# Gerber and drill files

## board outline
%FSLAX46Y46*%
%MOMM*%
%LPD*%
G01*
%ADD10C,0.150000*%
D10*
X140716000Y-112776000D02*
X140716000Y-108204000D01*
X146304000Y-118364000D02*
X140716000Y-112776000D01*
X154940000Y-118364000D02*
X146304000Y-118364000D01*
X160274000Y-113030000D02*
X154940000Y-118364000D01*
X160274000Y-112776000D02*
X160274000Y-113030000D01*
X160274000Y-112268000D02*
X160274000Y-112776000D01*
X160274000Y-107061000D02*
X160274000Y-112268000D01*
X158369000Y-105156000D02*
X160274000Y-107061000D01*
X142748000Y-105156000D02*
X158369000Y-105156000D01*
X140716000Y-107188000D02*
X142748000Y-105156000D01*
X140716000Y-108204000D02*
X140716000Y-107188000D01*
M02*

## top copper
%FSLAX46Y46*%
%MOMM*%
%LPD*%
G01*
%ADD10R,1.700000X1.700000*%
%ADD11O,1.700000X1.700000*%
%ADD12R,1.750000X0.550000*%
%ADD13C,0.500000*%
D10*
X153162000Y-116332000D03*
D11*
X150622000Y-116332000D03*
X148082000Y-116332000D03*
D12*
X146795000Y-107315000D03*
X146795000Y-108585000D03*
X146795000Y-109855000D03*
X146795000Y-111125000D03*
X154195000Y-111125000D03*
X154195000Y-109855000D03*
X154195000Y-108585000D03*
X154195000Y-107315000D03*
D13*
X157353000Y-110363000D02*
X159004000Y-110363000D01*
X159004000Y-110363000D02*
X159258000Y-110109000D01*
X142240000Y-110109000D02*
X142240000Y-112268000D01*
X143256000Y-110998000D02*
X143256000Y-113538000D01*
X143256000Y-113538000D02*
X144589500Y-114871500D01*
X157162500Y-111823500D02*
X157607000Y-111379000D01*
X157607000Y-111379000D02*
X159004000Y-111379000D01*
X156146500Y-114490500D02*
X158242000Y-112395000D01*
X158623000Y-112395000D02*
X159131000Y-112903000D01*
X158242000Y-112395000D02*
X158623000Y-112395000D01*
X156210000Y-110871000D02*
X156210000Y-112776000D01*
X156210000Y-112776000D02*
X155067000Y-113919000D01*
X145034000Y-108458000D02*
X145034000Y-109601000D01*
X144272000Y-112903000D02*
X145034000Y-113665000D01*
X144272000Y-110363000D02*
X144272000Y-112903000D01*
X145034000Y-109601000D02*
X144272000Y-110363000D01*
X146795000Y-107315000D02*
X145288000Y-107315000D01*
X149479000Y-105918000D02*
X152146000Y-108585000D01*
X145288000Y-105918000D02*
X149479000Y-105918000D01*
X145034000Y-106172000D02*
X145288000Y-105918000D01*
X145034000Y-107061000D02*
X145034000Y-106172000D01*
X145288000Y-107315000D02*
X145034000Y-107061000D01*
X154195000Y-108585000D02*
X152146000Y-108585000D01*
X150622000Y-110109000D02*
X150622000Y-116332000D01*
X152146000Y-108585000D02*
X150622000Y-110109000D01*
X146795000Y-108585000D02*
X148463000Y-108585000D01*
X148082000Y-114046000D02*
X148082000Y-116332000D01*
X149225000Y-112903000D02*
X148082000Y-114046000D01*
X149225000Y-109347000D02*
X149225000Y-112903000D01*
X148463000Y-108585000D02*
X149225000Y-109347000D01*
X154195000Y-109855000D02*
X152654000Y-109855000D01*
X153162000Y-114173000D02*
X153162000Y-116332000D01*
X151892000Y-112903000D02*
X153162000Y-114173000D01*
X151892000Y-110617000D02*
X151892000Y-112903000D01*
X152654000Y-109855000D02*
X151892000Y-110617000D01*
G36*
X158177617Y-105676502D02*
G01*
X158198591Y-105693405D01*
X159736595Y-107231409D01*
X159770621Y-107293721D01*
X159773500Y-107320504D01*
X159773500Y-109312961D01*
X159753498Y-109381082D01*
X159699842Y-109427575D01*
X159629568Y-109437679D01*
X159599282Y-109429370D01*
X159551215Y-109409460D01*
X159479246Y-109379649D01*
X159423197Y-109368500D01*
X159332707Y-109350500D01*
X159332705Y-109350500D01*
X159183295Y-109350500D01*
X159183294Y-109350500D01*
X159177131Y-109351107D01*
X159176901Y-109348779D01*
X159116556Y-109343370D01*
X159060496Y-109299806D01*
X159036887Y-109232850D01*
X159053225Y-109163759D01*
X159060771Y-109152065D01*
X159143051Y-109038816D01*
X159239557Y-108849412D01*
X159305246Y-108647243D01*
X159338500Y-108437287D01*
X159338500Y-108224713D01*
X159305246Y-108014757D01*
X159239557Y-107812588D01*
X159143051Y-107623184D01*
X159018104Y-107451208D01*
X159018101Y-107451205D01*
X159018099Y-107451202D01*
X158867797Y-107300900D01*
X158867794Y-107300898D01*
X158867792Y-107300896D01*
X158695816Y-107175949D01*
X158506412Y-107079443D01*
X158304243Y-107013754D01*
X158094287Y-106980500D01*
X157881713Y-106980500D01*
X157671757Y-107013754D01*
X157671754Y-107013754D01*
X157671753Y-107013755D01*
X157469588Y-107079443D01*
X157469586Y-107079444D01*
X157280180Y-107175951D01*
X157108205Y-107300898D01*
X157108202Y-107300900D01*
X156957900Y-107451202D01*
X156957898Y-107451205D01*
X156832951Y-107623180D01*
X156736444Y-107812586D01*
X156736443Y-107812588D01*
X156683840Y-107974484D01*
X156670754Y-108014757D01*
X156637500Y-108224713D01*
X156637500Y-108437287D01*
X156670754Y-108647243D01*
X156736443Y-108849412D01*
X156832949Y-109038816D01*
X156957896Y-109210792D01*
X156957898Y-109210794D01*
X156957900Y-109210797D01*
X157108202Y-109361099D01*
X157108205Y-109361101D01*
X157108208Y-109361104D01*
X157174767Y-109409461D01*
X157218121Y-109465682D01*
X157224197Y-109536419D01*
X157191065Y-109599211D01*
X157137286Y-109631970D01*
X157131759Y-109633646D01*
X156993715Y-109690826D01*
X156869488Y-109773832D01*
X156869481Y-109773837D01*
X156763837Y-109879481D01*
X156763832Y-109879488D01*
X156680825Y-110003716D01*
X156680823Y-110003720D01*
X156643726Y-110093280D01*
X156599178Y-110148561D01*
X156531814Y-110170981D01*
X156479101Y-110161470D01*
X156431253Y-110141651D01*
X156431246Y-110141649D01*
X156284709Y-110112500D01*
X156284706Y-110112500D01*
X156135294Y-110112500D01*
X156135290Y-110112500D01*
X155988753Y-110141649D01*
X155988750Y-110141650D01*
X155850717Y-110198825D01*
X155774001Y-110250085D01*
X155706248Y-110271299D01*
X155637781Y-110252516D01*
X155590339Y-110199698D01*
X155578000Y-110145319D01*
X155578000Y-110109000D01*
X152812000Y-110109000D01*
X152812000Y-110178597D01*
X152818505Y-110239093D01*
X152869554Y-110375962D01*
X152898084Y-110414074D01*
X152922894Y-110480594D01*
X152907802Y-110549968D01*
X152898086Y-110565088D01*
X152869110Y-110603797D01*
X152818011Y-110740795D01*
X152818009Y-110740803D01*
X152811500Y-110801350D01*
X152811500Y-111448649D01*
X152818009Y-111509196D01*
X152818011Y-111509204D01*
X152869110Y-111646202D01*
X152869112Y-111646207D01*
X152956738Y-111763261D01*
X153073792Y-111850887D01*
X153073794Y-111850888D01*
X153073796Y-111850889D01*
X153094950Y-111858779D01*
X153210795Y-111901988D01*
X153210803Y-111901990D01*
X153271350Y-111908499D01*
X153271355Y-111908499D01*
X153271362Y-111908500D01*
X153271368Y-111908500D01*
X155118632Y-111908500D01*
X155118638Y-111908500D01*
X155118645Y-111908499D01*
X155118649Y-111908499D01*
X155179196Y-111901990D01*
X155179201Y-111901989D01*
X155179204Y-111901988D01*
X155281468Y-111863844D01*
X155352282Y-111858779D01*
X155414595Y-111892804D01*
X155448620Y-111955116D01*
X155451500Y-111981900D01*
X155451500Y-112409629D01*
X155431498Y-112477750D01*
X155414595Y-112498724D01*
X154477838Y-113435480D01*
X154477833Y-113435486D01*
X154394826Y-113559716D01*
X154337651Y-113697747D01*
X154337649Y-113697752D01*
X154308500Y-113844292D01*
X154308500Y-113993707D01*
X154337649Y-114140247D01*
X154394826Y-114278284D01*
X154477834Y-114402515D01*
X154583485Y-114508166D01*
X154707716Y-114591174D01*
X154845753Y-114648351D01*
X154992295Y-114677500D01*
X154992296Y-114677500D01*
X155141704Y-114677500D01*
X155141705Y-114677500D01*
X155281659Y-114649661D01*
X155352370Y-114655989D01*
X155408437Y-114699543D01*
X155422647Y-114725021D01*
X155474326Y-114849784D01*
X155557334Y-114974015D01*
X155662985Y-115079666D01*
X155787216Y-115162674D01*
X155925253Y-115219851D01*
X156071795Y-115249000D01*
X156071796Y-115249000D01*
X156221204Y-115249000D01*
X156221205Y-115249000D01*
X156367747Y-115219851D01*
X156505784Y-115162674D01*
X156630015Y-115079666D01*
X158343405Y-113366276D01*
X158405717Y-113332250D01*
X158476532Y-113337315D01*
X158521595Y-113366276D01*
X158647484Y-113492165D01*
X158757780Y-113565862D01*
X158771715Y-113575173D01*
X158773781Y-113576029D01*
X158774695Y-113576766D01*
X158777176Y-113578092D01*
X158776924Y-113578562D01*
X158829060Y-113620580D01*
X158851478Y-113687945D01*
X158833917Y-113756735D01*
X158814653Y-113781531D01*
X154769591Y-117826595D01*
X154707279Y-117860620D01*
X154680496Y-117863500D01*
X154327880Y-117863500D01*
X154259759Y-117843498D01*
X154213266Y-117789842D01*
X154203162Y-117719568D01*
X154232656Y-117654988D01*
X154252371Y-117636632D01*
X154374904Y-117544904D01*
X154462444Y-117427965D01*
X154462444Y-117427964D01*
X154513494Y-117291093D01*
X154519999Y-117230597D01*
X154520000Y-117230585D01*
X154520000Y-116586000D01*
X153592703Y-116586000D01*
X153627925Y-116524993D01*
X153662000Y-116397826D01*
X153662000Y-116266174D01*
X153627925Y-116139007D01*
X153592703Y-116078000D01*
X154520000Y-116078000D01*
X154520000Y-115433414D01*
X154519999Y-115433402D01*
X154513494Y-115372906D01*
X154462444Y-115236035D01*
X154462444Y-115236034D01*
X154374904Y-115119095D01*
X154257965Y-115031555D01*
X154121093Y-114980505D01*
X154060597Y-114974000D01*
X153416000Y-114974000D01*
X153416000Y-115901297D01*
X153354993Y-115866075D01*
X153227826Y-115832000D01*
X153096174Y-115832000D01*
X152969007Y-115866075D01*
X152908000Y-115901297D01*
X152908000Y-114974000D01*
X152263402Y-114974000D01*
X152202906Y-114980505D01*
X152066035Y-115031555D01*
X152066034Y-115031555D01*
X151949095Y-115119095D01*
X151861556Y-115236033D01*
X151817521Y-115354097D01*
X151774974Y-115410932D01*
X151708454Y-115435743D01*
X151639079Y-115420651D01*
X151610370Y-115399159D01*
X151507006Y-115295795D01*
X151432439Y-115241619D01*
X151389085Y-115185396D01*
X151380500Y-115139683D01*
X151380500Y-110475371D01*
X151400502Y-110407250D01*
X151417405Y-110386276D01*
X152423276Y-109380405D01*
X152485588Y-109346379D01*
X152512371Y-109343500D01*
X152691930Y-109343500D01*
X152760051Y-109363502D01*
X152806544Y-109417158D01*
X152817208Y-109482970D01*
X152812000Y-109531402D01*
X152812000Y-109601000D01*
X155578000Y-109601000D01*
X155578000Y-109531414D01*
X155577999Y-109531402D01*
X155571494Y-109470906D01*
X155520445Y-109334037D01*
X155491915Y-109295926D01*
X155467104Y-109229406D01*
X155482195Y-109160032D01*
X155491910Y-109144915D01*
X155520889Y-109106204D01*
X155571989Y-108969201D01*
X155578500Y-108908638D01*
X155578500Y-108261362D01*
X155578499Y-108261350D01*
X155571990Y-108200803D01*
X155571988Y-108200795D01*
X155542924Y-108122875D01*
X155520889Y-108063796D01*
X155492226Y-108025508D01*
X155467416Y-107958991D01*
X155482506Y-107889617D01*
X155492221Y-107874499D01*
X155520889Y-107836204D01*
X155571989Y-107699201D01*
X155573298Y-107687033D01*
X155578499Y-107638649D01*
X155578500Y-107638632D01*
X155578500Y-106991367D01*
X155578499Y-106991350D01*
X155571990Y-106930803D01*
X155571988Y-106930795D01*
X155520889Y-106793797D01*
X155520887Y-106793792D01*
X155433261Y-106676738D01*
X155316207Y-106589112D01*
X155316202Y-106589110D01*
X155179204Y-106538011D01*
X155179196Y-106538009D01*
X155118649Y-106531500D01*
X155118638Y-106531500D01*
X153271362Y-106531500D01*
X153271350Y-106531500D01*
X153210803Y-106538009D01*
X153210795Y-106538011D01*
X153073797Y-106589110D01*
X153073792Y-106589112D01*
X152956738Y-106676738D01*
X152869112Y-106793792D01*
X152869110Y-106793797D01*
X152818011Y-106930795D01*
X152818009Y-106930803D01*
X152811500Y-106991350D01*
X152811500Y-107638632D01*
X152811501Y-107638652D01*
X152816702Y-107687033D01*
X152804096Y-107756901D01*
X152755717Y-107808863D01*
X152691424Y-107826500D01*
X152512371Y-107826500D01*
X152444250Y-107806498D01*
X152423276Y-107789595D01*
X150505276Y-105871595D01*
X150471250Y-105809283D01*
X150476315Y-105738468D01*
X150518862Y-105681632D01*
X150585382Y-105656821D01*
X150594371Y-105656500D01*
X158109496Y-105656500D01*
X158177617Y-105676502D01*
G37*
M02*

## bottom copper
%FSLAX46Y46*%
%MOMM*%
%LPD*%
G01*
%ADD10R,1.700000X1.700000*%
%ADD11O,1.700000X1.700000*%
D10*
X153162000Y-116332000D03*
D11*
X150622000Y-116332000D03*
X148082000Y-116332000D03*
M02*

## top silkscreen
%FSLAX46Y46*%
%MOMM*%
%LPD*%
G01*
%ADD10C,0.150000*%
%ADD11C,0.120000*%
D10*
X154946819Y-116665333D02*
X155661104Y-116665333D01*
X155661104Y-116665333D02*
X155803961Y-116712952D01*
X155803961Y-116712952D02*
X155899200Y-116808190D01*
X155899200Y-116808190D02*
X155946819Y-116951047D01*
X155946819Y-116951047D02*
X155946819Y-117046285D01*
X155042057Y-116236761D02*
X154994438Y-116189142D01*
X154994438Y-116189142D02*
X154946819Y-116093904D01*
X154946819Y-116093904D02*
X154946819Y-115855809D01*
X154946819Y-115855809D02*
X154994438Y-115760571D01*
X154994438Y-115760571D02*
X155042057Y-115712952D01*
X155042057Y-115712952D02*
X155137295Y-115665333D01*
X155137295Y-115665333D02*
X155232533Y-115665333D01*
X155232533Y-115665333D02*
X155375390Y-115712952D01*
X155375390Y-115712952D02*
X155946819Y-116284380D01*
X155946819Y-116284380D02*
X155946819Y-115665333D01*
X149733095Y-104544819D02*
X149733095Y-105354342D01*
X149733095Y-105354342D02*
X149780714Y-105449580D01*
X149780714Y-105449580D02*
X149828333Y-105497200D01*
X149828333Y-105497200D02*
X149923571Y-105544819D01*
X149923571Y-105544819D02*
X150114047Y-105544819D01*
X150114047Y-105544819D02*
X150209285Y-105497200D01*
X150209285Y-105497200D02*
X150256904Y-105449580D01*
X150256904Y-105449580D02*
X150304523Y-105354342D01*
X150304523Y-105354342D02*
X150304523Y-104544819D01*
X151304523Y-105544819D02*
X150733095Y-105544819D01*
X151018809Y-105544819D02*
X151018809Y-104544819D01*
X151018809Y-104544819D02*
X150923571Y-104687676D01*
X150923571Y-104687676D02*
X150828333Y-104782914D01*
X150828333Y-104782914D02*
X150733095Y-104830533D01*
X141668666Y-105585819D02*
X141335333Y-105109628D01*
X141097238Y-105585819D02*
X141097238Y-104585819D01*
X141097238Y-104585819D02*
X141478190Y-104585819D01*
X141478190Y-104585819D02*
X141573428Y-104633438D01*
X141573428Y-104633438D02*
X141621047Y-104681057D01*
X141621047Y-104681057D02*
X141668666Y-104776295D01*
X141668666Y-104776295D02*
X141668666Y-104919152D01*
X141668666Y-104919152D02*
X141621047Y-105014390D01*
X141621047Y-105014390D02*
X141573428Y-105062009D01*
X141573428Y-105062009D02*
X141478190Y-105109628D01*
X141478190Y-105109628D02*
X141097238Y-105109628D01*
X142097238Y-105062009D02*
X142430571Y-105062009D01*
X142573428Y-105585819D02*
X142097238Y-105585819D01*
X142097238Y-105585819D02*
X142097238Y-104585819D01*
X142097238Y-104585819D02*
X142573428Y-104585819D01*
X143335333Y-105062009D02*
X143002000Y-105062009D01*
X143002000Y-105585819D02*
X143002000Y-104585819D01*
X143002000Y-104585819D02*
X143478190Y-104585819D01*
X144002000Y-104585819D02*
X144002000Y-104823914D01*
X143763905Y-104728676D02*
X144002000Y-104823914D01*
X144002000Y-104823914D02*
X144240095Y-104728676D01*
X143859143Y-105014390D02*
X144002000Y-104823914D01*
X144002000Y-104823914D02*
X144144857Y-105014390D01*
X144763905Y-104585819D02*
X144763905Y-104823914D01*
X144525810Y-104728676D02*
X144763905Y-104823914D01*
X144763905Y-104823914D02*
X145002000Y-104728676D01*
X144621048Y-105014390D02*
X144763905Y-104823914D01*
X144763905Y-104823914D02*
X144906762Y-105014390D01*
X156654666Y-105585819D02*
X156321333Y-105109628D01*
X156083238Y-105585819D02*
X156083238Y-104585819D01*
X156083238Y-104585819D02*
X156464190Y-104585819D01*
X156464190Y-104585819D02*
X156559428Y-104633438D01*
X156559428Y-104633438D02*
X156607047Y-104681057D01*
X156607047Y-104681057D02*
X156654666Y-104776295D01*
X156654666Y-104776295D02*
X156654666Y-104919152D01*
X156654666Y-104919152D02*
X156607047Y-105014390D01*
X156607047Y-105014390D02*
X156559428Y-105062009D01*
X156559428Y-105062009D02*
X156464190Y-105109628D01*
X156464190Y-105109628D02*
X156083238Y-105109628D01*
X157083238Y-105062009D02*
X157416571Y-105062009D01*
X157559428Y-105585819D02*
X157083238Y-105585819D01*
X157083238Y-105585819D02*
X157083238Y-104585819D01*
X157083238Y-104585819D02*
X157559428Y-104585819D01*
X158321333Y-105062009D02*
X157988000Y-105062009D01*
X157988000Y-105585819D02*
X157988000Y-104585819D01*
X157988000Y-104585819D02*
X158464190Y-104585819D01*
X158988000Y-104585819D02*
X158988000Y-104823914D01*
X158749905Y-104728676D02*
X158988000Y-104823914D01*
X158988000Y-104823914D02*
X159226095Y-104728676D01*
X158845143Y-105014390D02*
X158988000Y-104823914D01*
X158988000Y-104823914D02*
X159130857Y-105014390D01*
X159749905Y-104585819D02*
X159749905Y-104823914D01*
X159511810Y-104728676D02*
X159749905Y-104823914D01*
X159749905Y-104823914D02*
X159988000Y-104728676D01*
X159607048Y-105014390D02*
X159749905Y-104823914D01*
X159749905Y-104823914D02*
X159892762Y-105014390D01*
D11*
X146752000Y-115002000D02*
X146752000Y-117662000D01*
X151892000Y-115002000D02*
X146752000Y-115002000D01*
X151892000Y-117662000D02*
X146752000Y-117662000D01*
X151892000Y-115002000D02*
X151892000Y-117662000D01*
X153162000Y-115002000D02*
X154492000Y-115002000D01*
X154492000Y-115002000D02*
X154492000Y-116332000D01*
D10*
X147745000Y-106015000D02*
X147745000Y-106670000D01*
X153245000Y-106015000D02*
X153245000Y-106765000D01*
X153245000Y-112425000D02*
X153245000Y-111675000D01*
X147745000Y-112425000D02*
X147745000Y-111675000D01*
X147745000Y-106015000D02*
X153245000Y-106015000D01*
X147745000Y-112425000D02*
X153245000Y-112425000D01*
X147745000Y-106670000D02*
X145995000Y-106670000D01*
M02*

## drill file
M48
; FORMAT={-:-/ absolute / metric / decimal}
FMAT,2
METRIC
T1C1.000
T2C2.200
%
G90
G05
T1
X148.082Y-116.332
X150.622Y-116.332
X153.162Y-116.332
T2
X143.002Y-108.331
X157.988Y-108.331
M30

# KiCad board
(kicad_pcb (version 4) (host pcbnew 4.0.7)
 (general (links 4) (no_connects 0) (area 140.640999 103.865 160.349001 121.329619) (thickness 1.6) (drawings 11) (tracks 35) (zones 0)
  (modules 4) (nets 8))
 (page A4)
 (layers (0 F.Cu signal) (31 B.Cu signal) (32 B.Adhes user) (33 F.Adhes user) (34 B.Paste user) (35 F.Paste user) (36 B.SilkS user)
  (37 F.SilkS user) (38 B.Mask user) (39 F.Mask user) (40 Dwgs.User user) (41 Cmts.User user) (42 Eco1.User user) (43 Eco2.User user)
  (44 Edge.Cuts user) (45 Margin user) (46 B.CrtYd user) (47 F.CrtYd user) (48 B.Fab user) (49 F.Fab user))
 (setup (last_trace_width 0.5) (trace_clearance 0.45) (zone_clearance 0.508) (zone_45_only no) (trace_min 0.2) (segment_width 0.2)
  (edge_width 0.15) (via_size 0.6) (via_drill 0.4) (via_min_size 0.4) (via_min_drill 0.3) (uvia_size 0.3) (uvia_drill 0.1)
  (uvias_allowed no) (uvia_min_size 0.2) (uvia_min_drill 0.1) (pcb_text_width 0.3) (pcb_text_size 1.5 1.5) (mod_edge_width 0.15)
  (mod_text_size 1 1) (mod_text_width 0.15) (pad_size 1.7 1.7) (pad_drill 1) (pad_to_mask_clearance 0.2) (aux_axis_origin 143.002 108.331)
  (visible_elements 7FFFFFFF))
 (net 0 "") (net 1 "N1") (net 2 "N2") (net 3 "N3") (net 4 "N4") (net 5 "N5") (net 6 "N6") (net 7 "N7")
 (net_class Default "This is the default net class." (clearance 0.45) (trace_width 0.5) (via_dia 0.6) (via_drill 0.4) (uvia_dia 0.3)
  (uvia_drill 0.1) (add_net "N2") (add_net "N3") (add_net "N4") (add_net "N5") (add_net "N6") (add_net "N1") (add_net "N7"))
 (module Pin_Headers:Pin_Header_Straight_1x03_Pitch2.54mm (layer F.Cu) (at 153.162 116.332 270)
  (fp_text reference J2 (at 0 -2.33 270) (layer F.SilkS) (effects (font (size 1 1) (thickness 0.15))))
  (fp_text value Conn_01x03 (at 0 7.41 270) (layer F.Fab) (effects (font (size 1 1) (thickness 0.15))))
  (fp_line (start -1.33 6.41) (end 1.33 6.41) (layer F.SilkS) (width 0.12))
  (fp_line (start -1.33 1.27) (end -1.33 6.41) (layer F.SilkS) (width 0.12))
  (fp_line (start 1.33 1.27) (end 1.33 6.41) (layer F.SilkS) (width 0.12))
  (fp_line (start -1.33 1.27) (end 1.33 1.27) (layer F.SilkS) (width 0.12))
  (fp_line (start -1.33 0) (end -1.33 -1.33) (layer F.SilkS) (width 0.12))
  (fp_line (start -1.33 -1.33) (end 0 -1.33) (layer F.SilkS) (width 0.12))
  (pad 2 thru_hole rect (at 0 0 270) (size 1.7 1.7) (drill 1) (layers *.Cu *.Mask) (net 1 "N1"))
  (pad 1 thru_hole oval (at 0 2.54 270) (size 1.7 1.7) (drill 1) (layers *.Cu *.Mask) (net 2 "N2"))
  (pad 3 thru_hole oval (at 0 5.08 270) (size 1.7 1.7) (drill 1) (layers *.Cu *.Mask) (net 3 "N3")))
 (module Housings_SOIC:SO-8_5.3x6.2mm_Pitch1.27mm (layer F.Cu) (at 150.495 109.22)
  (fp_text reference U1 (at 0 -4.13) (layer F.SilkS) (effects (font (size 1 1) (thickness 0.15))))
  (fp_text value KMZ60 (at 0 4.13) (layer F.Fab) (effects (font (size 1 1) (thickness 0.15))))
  (fp_line (start -2.75 -3.205) (end -2.75 -2.55) (layer F.SilkS) (width 0.15))
  (fp_line (start 2.75 -3.205) (end 2.75 -2.455) (layer F.SilkS) (width 0.15))
  (fp_line (start 2.75 3.205) (end 2.75 2.455) (layer F.SilkS) (width 0.15))
  (fp_line (start -2.75 3.205) (end -2.75 2.455) (layer F.SilkS) (width 0.15))
  (fp_line (start -2.75 -3.205) (end 2.75 -3.205) (layer F.SilkS) (width 0.15))
  (fp_line (start -2.75 3.205) (end 2.75 3.205) (layer F.SilkS) (width 0.15))
  (fp_line (start -2.75 -2.55) (end -4.5 -2.55) (layer F.SilkS) (width 0.15))
  (pad 1 smd rect (at -3.7 -1.905) (size 1.75 0.55) (layers F.Cu F.Paste F.Mask) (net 2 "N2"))
  (pad 2 smd rect (at -3.7 -0.635) (size 1.75 0.55) (layers F.Cu F.Paste F.Mask) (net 3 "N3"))
  (pad 3 smd rect (at -3.7 0.635) (size 1.75 0.55) (layers F.Cu F.Paste F.Mask) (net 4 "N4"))
  (pad 4 smd rect (at -3.7 1.905) (size 1.75 0.55) (layers F.Cu F.Paste F.Mask) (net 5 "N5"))
  (pad 5 smd rect (at 3.7 1.905) (size 1.75 0.55) (layers F.Cu F.Paste F.Mask) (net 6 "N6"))
  (pad 6 smd rect (at 3.7 0.635) (size 1.75 0.55) (layers F.Cu F.Paste F.Mask) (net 1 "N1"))
  (pad 7 smd rect (at 3.7 -0.635) (size 1.75 0.55) (layers F.Cu F.Paste F.Mask) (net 2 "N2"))
  (pad 8 smd rect (at 3.7 -1.905) (size 1.75 0.55) (layers F.Cu F.Paste F.Mask) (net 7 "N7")))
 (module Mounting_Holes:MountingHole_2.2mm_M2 (layer F.Cu) (at 143.002 108.331)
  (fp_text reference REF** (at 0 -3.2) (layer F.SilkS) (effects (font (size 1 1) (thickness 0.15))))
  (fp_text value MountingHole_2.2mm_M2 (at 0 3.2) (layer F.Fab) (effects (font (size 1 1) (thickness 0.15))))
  (pad 1 np_thru_hole circle (at 0 0) (size 2.2 2.2) (drill 2.2) (layers *.Cu *.Mask)))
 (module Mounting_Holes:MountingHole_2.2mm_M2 (layer F.Cu) (at 157.988 108.331)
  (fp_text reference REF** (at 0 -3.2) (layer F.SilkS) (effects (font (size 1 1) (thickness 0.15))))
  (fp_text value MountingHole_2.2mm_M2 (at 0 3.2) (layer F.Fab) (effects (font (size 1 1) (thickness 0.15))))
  (pad 1 np_thru_hole circle (at 0 0) (size 2.2 2.2) (drill 2.2) (layers *.Cu *.Mask)))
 (gr_line (start 140.716 112.776) (end 140.716 108.204) (angle 90) (layer Edge.Cuts) (width 0.15))
 (gr_line (start 146.304 118.364) (end 140.716 112.776) (angle 90) (layer Edge.Cuts) (width 0.15))
 (gr_line (start 154.94 118.364) (end 146.304 118.364) (angle 90) (layer Edge.Cuts) (width 0.15))
 (gr_line (start 160.274 113.03) (end 154.94 118.364) (angle 90) (layer Edge.Cuts) (width 0.15))
 (gr_line (start 160.274 112.776) (end 160.274 113.03) (angle 90) (layer Edge.Cuts) (width 0.15))
 (gr_line (start 160.274 112.268) (end 160.274 112.776) (angle 90) (layer Edge.Cuts) (width 0.15))
 (gr_line (start 160.274 107.061) (end 160.274 112.268) (angle 90) (layer Edge.Cuts) (width 0.15))
 (gr_line (start 158.369 105.156) (end 160.274 107.061) (angle 90) (layer Edge.Cuts) (width 0.15))
 (gr_line (start 142.748 105.156) (end 158.369 105.156) (angle 90) (layer Edge.Cuts) (width 0.15))
 (gr_line (start 140.716 107.188) (end 142.748 105.156) (angle 90) (layer Edge.Cuts) (width 0.15))
 (gr_line (start 140.716 108.204) (end 140.716 107.188) (angle 90) (layer Edge.Cuts) (width 0.15))
 (segment (start 157.353 110.363) (end 159.004 110.363) (width 0.5) (layer F.Cu) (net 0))
 (segment (start 159.004 110.363) (end 159.258 110.109) (width 0.5) (layer F.Cu) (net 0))
 (segment (start 142.24 110.109) (end 142.24 112.268) (width 0.5) (layer F.Cu) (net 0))
 (segment (start 143.256 110.998) (end 143.256 113.538) (width 0.5) (layer F.Cu) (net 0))
 (segment (start 143.256 113.538) (end 144.5895 114.8715) (width 0.5) (layer F.Cu) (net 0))
 (segment (start 157.1625 111.8235) (end 157.607 111.379) (width 0.5) (layer F.Cu) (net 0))
 (segment (start 157.607 111.379) (end 159.004 111.379) (width 0.5) (layer F.Cu) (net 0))
 (segment (start 156.1465 114.4905) (end 158.242 112.395) (width 0.5) (layer F.Cu) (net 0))
 (segment (start 158.623 112.395) (end 159.131 112.903) (width 0.5) (layer F.Cu) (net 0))
 (segment (start 158.242 112.395) (end 158.623 112.395) (width 0.5) (layer F.Cu) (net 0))
 (segment (start 156.21 110.871) (end 156.21 112.776) (width 0.5) (layer F.Cu) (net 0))
 (segment (start 156.21 112.776) (end 155.067 113.919) (width 0.5) (layer F.Cu) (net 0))
 (segment (start 145.034 108.458) (end 145.034 109.601) (width 0.5) (layer F.Cu) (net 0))
 (segment (start 144.272 112.903) (end 145.034 113.665) (width 0.5) (layer F.Cu) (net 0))
 (segment (start 144.272 110.363) (end 144.272 112.903) (width 0.5) (layer F.Cu) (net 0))
 (segment (start 145.034 109.601) (end 144.272 110.363) (width 0.5) (layer F.Cu) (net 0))
 (segment (start 146.795 107.315) (end 145.288 107.315) (width 0.5) (layer F.Cu) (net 2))
 (segment (start 149.479 105.918) (end 152.146 108.585) (width 0.5) (layer F.Cu) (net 2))
 (segment (start 145.288 105.918) (end 149.479 105.918) (width 0.5) (layer F.Cu) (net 2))
 (segment (start 145.034 106.172) (end 145.288 105.918) (width 0.5) (layer F.Cu) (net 2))
 (segment (start 145.034 107.061) (end 145.034 106.172) (width 0.5) (layer F.Cu) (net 2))
 (segment (start 145.288 107.315) (end 145.034 107.061) (width 0.5) (layer F.Cu) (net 2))
 (segment (start 154.195 108.585) (end 152.146 108.585) (width 0.5) (layer F.Cu) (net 2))
 (segment (start 150.622 110.109) (end 150.622 116.332) (width 0.5) (layer F.Cu) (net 2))
 (segment (start 152.146 108.585) (end 150.622 110.109) (width 0.5) (layer F.Cu) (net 2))
 (segment (start 146.795 108.585) (end 148.463 108.585) (width 0.5) (layer F.Cu) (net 3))
 (segment (start 148.082 114.046) (end 148.082 116.332) (width 0.5) (layer F.Cu) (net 3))
 (segment (start 149.225 112.903) (end 148.082 114.046) (width 0.5) (layer F.Cu) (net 3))
 (segment (start 149.225 109.347) (end 149.225 112.903) (width 0.5) (layer F.Cu) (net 3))
 (segment (start 148.463 108.585) (end 149.225 109.347) (width 0.5) (layer F.Cu) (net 3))
 (segment (start 154.195 109.855) (end 152.654 109.855) (width 0.5) (layer F.Cu) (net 1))
 (segment (start 153.162 114.173) (end 153.162 116.332) (width 0.5) (layer F.Cu) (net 1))
 (segment (start 151.892 112.903) (end 153.162 114.173) (width 0.5) (layer F.Cu) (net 1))
 (segment (start 151.892 110.617) (end 151.892 112.903) (width 0.5) (layer F.Cu) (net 1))
 (segment (start 152.654 109.855) (end 151.892 110.617) (width 0.5) (layer F.Cu) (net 1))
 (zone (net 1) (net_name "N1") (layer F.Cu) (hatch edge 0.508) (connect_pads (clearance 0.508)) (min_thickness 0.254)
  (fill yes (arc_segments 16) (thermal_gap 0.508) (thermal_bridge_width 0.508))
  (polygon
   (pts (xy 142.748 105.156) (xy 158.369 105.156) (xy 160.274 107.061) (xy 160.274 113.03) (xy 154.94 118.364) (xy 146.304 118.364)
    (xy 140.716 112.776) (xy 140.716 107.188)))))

